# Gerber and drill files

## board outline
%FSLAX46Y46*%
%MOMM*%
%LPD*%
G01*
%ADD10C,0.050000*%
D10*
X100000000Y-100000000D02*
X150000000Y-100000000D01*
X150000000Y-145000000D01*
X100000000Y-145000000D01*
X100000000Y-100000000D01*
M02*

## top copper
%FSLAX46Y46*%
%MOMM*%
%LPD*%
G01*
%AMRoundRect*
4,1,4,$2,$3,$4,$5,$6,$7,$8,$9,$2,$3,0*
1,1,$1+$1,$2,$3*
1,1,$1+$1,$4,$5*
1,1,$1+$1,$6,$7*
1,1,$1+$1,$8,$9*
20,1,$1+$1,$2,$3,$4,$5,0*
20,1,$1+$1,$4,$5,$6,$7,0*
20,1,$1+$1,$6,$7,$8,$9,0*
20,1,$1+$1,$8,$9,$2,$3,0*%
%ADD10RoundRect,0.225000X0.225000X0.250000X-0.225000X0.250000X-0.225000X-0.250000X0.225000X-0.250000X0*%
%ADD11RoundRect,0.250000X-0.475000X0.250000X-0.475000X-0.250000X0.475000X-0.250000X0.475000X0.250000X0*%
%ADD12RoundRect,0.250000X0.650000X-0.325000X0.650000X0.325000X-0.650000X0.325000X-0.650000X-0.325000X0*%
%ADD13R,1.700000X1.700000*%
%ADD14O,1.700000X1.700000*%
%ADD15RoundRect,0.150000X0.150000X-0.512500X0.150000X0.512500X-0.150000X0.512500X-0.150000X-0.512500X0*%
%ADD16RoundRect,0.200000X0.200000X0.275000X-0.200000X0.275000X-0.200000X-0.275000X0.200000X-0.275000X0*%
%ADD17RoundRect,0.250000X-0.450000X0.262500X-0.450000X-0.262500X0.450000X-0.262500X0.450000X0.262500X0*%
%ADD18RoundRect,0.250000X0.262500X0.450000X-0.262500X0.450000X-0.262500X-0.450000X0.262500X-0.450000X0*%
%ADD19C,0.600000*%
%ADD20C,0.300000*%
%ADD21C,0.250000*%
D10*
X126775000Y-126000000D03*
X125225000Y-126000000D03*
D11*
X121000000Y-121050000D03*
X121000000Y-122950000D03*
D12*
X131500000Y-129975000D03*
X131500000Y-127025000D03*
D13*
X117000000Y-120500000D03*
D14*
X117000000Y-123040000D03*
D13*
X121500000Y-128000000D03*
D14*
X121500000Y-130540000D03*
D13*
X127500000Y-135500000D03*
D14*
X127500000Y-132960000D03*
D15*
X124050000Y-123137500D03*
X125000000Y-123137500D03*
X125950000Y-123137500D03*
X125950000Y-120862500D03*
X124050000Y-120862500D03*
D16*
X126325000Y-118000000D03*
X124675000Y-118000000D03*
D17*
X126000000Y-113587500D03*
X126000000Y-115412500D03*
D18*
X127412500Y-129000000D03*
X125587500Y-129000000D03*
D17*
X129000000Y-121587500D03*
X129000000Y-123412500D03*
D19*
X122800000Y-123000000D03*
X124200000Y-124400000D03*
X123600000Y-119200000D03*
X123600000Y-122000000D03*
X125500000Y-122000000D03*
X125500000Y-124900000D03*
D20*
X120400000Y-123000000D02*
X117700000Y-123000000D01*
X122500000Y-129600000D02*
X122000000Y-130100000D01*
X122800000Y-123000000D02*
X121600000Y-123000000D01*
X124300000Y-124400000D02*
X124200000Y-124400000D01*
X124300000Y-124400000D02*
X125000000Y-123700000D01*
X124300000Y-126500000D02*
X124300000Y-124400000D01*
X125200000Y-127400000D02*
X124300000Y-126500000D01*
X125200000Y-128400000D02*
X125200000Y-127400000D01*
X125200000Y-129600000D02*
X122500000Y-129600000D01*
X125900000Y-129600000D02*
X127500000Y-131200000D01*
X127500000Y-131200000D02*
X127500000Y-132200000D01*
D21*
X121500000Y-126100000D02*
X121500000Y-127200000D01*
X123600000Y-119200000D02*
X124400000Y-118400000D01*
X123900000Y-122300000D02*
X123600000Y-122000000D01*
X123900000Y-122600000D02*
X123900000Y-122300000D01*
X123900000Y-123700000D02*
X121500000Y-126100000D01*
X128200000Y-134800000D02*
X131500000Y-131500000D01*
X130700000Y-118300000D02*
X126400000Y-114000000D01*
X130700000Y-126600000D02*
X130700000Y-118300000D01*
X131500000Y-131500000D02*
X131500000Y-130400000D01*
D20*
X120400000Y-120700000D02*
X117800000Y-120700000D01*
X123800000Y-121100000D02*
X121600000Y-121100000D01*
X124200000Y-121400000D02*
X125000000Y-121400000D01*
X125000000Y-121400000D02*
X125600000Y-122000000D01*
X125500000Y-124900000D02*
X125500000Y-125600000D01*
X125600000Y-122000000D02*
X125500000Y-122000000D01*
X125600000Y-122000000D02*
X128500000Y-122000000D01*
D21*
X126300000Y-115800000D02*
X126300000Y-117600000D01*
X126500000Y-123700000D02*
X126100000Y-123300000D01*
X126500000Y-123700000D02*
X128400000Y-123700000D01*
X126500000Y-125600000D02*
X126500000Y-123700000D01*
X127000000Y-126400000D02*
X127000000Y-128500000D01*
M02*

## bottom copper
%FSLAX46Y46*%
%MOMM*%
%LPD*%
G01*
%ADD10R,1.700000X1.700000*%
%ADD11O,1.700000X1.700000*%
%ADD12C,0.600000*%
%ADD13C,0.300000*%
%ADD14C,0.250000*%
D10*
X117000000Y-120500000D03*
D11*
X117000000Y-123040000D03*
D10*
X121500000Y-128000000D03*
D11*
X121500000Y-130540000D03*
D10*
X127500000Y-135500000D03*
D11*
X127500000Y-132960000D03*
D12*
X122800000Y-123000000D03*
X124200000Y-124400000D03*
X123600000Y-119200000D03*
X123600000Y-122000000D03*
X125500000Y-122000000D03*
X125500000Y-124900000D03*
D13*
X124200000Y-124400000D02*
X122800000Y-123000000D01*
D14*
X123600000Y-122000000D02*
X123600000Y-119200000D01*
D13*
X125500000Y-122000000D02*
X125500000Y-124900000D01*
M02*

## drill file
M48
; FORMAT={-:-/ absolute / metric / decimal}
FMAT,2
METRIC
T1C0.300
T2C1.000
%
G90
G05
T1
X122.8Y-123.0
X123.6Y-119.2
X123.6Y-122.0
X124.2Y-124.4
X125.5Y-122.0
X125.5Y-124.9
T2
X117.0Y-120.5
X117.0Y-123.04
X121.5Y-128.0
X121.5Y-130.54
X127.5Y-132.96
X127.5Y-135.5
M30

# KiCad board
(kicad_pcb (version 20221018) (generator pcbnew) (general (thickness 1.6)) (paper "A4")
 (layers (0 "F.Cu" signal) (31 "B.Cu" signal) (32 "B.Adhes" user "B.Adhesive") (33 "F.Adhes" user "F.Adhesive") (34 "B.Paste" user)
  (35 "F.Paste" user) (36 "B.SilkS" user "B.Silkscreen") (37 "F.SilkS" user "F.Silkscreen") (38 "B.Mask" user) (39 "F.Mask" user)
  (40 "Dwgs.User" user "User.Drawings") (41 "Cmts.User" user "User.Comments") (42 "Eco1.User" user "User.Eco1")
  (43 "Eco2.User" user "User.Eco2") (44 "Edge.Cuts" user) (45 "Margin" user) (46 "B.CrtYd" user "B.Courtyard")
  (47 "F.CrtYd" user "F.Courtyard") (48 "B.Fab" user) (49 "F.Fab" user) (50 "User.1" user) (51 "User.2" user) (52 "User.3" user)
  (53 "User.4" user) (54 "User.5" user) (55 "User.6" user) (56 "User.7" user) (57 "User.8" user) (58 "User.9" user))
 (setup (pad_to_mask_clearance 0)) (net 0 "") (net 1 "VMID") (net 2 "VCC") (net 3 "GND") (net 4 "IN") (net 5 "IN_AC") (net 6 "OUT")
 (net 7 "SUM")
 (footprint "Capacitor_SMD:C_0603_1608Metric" (layer "F.Cu") (at 126 126 180)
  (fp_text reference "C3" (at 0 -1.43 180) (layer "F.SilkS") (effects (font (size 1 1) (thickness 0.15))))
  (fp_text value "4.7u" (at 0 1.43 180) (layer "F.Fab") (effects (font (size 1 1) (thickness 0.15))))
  (pad "1" smd roundrect (at -0.775 0 180) (size 0.9 0.95) (layers "F.Cu" "F.Paste" "F.Mask") (roundrect_rratio 0.25) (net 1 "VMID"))
  (pad "2" smd roundrect (at 0.775 0 180) (size 0.9 0.95) (layers "F.Cu" "F.Paste" "F.Mask") (roundrect_rratio 0.25) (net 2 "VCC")))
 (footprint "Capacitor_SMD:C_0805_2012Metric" (layer "F.Cu") (at 121 122 -90)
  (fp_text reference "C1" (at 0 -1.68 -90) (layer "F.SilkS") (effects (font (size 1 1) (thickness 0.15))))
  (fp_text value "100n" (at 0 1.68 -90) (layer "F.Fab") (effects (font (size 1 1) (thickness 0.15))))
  (pad "1" smd roundrect (at -0.95 0 270) (size 1 1.45) (layers "F.Cu" "F.Paste" "F.Mask") (roundrect_rratio 0.25) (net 2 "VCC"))
  (pad "2" smd roundrect (at 0.95 0 270) (size 1 1.45) (layers "F.Cu" "F.Paste" "F.Mask") (roundrect_rratio 0.25) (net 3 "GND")))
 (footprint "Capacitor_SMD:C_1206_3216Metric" (layer "F.Cu") (at 131.5 128.5 90)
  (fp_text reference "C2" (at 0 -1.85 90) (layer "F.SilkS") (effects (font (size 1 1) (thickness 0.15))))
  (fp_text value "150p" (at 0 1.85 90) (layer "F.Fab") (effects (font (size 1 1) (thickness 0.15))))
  (pad "1" smd roundrect (at -1.475 0 90) (size 1.15 1.8) (layers "F.Cu" "F.Paste" "F.Mask") (roundrect_rratio 0.217391) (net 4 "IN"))
  (pad "2" smd roundrect (at 1.475 0 90) (size 1.15 1.8) (layers "F.Cu" "F.Paste" "F.Mask") (roundrect_rratio 0.217391) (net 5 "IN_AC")))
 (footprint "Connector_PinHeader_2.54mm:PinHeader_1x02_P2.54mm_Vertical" (layer "F.Cu") (at 117 120.5)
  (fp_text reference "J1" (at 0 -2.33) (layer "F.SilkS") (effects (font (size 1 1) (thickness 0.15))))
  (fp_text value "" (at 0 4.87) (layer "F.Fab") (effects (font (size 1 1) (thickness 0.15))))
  (pad "1" thru_hole rect (at 0 0) (size 1.7 1.7) (drill 1) (layers "*.Cu" "*.Mask") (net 2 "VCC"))
  (pad "2" thru_hole oval (at 0 2.54) (size 1.7 1.7) (drill 1) (layers "*.Cu" "*.Mask") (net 3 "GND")))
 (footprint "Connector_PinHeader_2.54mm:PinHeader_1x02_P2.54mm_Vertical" (layer "F.Cu") (at 121.5 128)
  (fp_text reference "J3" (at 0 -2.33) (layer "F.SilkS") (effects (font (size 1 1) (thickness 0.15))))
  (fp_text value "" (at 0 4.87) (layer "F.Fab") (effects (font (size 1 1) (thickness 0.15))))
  (pad "1" thru_hole rect (at 0 0) (size 1.7 1.7) (drill 1) (layers "*.Cu" "*.Mask") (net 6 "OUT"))
  (pad "2" thru_hole oval (at 0 2.54) (size 1.7 1.7) (drill 1) (layers "*.Cu" "*.Mask") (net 3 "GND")))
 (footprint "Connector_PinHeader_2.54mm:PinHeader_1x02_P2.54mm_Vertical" (layer "F.Cu") (at 127.5 135.5 180)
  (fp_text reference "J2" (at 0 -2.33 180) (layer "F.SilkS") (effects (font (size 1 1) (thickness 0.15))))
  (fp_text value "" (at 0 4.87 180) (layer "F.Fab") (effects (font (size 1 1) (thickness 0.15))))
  (pad "1" thru_hole rect (at 0 0 180) (size 1.7 1.7) (drill 1) (layers "*.Cu" "*.Mask") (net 4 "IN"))
  (pad "2" thru_hole oval (at 0 2.54 180) (size 1.7 1.7) (drill 1) (layers "*.Cu" "*.Mask") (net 3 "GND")))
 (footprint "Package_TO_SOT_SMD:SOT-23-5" (layer "F.Cu") (at 125 122 90)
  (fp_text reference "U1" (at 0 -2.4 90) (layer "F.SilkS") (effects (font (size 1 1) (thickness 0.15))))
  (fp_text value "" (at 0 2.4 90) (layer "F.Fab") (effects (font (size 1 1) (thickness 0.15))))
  (pad "1" smd roundrect (at -1.1375 -0.95 90) (size 1.325 0.6) (layers "F.Cu" "F.Paste" "F.Mask") (roundrect_rratio 0.25) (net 6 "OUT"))
  (pad "2" smd roundrect (at -1.1375 0 90) (size 1.325 0.6) (layers "F.Cu" "F.Paste" "F.Mask") (roundrect_rratio 0.25) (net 3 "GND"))
  (pad "3" smd roundrect (at -1.1375 0.95 90) (size 1.325 0.6) (layers "F.Cu" "F.Paste" "F.Mask") (roundrect_rratio 0.25) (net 1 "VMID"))
  (pad "4" smd roundrect (at 1.1375 0.95 90) (size 1.325 0.6) (layers "F.Cu" "F.Paste" "F.Mask") (roundrect_rratio 0.25))
  (pad "5" smd roundrect (at 1.1375 -0.95 90) (size 1.325 0.6) (layers "F.Cu" "F.Paste" "F.Mask") (roundrect_rratio 0.25) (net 2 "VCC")))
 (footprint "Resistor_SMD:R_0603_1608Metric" (layer "F.Cu") (at 125.5 118 180)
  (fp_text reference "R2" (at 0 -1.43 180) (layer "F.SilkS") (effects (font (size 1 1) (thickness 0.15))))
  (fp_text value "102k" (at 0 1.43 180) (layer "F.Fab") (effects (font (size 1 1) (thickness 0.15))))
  (pad "1" smd roundrect (at -0.825 0 180) (size 0.8 0.95) (layers "F.Cu" "F.Paste" "F.Mask") (roundrect_rratio 0.25) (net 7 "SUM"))
  (pad "2" smd roundrect (at 0.825 0 180) (size 0.8 0.95) (layers "F.Cu" "F.Paste" "F.Mask") (roundrect_rratio 0.25) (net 6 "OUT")))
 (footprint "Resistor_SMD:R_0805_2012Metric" (layer "F.Cu") (at 126 114.5 -90)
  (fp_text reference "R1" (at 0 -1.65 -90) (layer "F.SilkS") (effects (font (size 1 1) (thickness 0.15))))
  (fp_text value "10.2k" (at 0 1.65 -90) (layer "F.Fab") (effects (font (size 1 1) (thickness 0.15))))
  (pad "1" smd roundrect (at -0.9125 0 270) (size 1.025 1.4) (layers "F.Cu" "F.Paste" "F.Mask") (roundrect_rratio 0.243902) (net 5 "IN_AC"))
  (pad "2" smd roundrect (at 0.9125 0 270) (size 1.025 1.4) (layers "F.Cu" "F.Paste" "F.Mask") (roundrect_rratio 0.243902) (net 7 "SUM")))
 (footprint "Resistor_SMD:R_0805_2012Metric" (layer "F.Cu") (at 126.5 129 180)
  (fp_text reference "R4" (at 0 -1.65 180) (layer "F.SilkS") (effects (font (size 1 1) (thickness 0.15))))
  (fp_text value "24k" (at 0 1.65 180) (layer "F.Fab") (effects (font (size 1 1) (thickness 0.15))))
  (pad "1" smd roundrect (at -0.9125 0 180) (size 1.025 1.4) (layers "F.Cu" "F.Paste" "F.Mask") (roundrect_rratio 0.243902) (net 1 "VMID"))
  (pad "2" smd roundrect (at 0.9125 0 180) (size 1.025 1.4) (layers "F.Cu" "F.Paste" "F.Mask") (roundrect_rratio 0.243902) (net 3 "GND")))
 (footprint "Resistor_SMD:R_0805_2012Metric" (layer "F.Cu") (at 129 122.5 -90)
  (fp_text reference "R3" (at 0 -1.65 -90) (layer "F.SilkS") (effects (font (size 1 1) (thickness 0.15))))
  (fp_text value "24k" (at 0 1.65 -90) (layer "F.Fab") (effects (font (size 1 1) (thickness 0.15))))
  (pad "1" smd roundrect (at -0.9125 0 270) (size 1.025 1.4) (layers "F.Cu" "F.Paste" "F.Mask") (roundrect_rratio 0.243902) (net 2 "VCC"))
  (pad "2" smd roundrect (at 0.9125 0 270) (size 1.025 1.4) (layers "F.Cu" "F.Paste" "F.Mask") (roundrect_rratio 0.243902) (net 1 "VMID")))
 (gr_rect (start 100 100) (end 150 145) (stroke (width 0.05) (type default)) (fill none) (layer "Edge.Cuts"))
 (segment (start 120.4 123) (end 117.7 123) (width 0.3) (layer "F.Cu") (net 3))
 (segment (start 122.5 129.6) (end 122 130.1) (width 0.3) (layer "F.Cu") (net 3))
 (segment (start 122.8 123) (end 121.6 123) (width 0.3) (layer "F.Cu") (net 3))
 (segment (start 124.3 124.4) (end 124.2 124.4) (width 0.3) (layer "F.Cu") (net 3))
 (segment (start 124.3 124.4) (end 125 123.7) (width 0.3) (layer "F.Cu") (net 3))
 (segment (start 124.3 126.5) (end 124.3 124.4) (width 0.3) (layer "F.Cu") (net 3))
 (segment (start 125.2 127.4) (end 124.3 126.5) (width 0.3) (layer "F.Cu") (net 3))
 (segment (start 125.2 128.4) (end 125.2 127.4) (width 0.3) (layer "F.Cu") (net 3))
 (segment (start 125.2 129.6) (end 122.5 129.6) (width 0.3) (layer "F.Cu") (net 3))
 (segment (start 125.9 129.6) (end 127.5 131.2) (width 0.3) (layer "F.Cu") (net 3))
 (segment (start 127.5 131.2) (end 127.5 132.2) (width 0.3) (layer "F.Cu") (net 3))
 (via (at 122.8 123) (size 0.6) (drill 0.3) (layers "F.Cu" "B.Cu") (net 3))
 (via (at 124.2 124.4) (size 0.6) (drill 0.3) (layers "F.Cu" "B.Cu") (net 3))
 (segment (start 121.5 126.1) (end 121.5 127.2) (width 0.25) (layer "F.Cu") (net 6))
 (segment (start 123.6 119.2) (end 124.4 118.4) (width 0.25) (layer "F.Cu") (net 6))
 (segment (start 123.9 122.3) (end 123.6 122) (width 0.25) (layer "F.Cu") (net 6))
 (segment (start 123.9 122.6) (end 123.9 122.3) (width 0.25) (layer "F.Cu") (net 6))
 (segment (start 123.9 123.7) (end 121.5 126.1) (width 0.25) (layer "F.Cu") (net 6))
 (segment (start 124.2 124.4) (end 122.8 123) (width 0.3) (layer "B.Cu") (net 3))
 (segment (start 128.2 134.8) (end 131.5 131.5) (width 0.25) (layer "F.Cu") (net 4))
 (segment (start 130.7 118.3) (end 126.4 114) (width 0.25) (layer "F.Cu") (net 5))
 (segment (start 130.7 126.6) (end 130.7 118.3) (width 0.25) (layer "F.Cu") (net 5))
 (segment (start 131.5 131.5) (end 131.5 130.4) (width 0.25) (layer "F.Cu") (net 4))
 (via (at 123.6 119.2) (size 0.6) (drill 0.3) (layers "F.Cu" "B.Cu") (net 6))
 (via (at 123.6 122) (size 0.6) (drill 0.3) (layers "F.Cu" "B.Cu") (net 6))
 (segment (start 120.4 120.7) (end 117.8 120.7) (width 0.3) (layer "F.Cu") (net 2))
 (segment (start 123.6 122) (end 123.6 119.2) (width 0.25) (layer "B.Cu") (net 6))
 (segment (start 123.8 121.1) (end 121.6 121.1) (width 0.3) (layer "F.Cu") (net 2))
 (segment (start 124.2 121.4) (end 125 121.4) (width 0.3) (layer "F.Cu") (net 2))
 (segment (start 125 121.4) (end 125.6 122) (width 0.3) (layer "F.Cu") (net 2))
 (segment (start 125.5 124.9) (end 125.5 125.6) (width 0.3) (layer "F.Cu") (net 2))
 (segment (start 125.6 122) (end 125.5 122) (width 0.3) (layer "F.Cu") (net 2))
 (segment (start 125.6 122) (end 128.5 122) (width 0.3) (layer "F.Cu") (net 2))
 (segment (start 126.3 115.8) (end 126.3 117.6) (width 0.25) (layer "F.Cu") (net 7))
 (via (at 125.5 122) (size 0.6) (drill 0.3) (layers "F.Cu" "B.Cu") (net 2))
 (via (at 125.5 124.9) (size 0.6) (drill 0.3) (layers "F.Cu" "B.Cu") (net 2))
 (segment (start 125.5 122) (end 125.5 124.9) (width 0.3) (layer "B.Cu") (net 2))
 (segment (start 126.5 123.7) (end 126.1 123.3) (width 0.25) (layer "F.Cu") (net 1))
 (segment (start 126.5 123.7) (end 128.4 123.7) (width 0.25) (layer "F.Cu") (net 1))
 (segment (start 126.5 125.6) (end 126.5 123.7) (width 0.25) (layer "F.Cu") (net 1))
 (segment (start 127 126.4) (end 127 128.5) (width 0.25) (layer "F.Cu") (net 1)))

